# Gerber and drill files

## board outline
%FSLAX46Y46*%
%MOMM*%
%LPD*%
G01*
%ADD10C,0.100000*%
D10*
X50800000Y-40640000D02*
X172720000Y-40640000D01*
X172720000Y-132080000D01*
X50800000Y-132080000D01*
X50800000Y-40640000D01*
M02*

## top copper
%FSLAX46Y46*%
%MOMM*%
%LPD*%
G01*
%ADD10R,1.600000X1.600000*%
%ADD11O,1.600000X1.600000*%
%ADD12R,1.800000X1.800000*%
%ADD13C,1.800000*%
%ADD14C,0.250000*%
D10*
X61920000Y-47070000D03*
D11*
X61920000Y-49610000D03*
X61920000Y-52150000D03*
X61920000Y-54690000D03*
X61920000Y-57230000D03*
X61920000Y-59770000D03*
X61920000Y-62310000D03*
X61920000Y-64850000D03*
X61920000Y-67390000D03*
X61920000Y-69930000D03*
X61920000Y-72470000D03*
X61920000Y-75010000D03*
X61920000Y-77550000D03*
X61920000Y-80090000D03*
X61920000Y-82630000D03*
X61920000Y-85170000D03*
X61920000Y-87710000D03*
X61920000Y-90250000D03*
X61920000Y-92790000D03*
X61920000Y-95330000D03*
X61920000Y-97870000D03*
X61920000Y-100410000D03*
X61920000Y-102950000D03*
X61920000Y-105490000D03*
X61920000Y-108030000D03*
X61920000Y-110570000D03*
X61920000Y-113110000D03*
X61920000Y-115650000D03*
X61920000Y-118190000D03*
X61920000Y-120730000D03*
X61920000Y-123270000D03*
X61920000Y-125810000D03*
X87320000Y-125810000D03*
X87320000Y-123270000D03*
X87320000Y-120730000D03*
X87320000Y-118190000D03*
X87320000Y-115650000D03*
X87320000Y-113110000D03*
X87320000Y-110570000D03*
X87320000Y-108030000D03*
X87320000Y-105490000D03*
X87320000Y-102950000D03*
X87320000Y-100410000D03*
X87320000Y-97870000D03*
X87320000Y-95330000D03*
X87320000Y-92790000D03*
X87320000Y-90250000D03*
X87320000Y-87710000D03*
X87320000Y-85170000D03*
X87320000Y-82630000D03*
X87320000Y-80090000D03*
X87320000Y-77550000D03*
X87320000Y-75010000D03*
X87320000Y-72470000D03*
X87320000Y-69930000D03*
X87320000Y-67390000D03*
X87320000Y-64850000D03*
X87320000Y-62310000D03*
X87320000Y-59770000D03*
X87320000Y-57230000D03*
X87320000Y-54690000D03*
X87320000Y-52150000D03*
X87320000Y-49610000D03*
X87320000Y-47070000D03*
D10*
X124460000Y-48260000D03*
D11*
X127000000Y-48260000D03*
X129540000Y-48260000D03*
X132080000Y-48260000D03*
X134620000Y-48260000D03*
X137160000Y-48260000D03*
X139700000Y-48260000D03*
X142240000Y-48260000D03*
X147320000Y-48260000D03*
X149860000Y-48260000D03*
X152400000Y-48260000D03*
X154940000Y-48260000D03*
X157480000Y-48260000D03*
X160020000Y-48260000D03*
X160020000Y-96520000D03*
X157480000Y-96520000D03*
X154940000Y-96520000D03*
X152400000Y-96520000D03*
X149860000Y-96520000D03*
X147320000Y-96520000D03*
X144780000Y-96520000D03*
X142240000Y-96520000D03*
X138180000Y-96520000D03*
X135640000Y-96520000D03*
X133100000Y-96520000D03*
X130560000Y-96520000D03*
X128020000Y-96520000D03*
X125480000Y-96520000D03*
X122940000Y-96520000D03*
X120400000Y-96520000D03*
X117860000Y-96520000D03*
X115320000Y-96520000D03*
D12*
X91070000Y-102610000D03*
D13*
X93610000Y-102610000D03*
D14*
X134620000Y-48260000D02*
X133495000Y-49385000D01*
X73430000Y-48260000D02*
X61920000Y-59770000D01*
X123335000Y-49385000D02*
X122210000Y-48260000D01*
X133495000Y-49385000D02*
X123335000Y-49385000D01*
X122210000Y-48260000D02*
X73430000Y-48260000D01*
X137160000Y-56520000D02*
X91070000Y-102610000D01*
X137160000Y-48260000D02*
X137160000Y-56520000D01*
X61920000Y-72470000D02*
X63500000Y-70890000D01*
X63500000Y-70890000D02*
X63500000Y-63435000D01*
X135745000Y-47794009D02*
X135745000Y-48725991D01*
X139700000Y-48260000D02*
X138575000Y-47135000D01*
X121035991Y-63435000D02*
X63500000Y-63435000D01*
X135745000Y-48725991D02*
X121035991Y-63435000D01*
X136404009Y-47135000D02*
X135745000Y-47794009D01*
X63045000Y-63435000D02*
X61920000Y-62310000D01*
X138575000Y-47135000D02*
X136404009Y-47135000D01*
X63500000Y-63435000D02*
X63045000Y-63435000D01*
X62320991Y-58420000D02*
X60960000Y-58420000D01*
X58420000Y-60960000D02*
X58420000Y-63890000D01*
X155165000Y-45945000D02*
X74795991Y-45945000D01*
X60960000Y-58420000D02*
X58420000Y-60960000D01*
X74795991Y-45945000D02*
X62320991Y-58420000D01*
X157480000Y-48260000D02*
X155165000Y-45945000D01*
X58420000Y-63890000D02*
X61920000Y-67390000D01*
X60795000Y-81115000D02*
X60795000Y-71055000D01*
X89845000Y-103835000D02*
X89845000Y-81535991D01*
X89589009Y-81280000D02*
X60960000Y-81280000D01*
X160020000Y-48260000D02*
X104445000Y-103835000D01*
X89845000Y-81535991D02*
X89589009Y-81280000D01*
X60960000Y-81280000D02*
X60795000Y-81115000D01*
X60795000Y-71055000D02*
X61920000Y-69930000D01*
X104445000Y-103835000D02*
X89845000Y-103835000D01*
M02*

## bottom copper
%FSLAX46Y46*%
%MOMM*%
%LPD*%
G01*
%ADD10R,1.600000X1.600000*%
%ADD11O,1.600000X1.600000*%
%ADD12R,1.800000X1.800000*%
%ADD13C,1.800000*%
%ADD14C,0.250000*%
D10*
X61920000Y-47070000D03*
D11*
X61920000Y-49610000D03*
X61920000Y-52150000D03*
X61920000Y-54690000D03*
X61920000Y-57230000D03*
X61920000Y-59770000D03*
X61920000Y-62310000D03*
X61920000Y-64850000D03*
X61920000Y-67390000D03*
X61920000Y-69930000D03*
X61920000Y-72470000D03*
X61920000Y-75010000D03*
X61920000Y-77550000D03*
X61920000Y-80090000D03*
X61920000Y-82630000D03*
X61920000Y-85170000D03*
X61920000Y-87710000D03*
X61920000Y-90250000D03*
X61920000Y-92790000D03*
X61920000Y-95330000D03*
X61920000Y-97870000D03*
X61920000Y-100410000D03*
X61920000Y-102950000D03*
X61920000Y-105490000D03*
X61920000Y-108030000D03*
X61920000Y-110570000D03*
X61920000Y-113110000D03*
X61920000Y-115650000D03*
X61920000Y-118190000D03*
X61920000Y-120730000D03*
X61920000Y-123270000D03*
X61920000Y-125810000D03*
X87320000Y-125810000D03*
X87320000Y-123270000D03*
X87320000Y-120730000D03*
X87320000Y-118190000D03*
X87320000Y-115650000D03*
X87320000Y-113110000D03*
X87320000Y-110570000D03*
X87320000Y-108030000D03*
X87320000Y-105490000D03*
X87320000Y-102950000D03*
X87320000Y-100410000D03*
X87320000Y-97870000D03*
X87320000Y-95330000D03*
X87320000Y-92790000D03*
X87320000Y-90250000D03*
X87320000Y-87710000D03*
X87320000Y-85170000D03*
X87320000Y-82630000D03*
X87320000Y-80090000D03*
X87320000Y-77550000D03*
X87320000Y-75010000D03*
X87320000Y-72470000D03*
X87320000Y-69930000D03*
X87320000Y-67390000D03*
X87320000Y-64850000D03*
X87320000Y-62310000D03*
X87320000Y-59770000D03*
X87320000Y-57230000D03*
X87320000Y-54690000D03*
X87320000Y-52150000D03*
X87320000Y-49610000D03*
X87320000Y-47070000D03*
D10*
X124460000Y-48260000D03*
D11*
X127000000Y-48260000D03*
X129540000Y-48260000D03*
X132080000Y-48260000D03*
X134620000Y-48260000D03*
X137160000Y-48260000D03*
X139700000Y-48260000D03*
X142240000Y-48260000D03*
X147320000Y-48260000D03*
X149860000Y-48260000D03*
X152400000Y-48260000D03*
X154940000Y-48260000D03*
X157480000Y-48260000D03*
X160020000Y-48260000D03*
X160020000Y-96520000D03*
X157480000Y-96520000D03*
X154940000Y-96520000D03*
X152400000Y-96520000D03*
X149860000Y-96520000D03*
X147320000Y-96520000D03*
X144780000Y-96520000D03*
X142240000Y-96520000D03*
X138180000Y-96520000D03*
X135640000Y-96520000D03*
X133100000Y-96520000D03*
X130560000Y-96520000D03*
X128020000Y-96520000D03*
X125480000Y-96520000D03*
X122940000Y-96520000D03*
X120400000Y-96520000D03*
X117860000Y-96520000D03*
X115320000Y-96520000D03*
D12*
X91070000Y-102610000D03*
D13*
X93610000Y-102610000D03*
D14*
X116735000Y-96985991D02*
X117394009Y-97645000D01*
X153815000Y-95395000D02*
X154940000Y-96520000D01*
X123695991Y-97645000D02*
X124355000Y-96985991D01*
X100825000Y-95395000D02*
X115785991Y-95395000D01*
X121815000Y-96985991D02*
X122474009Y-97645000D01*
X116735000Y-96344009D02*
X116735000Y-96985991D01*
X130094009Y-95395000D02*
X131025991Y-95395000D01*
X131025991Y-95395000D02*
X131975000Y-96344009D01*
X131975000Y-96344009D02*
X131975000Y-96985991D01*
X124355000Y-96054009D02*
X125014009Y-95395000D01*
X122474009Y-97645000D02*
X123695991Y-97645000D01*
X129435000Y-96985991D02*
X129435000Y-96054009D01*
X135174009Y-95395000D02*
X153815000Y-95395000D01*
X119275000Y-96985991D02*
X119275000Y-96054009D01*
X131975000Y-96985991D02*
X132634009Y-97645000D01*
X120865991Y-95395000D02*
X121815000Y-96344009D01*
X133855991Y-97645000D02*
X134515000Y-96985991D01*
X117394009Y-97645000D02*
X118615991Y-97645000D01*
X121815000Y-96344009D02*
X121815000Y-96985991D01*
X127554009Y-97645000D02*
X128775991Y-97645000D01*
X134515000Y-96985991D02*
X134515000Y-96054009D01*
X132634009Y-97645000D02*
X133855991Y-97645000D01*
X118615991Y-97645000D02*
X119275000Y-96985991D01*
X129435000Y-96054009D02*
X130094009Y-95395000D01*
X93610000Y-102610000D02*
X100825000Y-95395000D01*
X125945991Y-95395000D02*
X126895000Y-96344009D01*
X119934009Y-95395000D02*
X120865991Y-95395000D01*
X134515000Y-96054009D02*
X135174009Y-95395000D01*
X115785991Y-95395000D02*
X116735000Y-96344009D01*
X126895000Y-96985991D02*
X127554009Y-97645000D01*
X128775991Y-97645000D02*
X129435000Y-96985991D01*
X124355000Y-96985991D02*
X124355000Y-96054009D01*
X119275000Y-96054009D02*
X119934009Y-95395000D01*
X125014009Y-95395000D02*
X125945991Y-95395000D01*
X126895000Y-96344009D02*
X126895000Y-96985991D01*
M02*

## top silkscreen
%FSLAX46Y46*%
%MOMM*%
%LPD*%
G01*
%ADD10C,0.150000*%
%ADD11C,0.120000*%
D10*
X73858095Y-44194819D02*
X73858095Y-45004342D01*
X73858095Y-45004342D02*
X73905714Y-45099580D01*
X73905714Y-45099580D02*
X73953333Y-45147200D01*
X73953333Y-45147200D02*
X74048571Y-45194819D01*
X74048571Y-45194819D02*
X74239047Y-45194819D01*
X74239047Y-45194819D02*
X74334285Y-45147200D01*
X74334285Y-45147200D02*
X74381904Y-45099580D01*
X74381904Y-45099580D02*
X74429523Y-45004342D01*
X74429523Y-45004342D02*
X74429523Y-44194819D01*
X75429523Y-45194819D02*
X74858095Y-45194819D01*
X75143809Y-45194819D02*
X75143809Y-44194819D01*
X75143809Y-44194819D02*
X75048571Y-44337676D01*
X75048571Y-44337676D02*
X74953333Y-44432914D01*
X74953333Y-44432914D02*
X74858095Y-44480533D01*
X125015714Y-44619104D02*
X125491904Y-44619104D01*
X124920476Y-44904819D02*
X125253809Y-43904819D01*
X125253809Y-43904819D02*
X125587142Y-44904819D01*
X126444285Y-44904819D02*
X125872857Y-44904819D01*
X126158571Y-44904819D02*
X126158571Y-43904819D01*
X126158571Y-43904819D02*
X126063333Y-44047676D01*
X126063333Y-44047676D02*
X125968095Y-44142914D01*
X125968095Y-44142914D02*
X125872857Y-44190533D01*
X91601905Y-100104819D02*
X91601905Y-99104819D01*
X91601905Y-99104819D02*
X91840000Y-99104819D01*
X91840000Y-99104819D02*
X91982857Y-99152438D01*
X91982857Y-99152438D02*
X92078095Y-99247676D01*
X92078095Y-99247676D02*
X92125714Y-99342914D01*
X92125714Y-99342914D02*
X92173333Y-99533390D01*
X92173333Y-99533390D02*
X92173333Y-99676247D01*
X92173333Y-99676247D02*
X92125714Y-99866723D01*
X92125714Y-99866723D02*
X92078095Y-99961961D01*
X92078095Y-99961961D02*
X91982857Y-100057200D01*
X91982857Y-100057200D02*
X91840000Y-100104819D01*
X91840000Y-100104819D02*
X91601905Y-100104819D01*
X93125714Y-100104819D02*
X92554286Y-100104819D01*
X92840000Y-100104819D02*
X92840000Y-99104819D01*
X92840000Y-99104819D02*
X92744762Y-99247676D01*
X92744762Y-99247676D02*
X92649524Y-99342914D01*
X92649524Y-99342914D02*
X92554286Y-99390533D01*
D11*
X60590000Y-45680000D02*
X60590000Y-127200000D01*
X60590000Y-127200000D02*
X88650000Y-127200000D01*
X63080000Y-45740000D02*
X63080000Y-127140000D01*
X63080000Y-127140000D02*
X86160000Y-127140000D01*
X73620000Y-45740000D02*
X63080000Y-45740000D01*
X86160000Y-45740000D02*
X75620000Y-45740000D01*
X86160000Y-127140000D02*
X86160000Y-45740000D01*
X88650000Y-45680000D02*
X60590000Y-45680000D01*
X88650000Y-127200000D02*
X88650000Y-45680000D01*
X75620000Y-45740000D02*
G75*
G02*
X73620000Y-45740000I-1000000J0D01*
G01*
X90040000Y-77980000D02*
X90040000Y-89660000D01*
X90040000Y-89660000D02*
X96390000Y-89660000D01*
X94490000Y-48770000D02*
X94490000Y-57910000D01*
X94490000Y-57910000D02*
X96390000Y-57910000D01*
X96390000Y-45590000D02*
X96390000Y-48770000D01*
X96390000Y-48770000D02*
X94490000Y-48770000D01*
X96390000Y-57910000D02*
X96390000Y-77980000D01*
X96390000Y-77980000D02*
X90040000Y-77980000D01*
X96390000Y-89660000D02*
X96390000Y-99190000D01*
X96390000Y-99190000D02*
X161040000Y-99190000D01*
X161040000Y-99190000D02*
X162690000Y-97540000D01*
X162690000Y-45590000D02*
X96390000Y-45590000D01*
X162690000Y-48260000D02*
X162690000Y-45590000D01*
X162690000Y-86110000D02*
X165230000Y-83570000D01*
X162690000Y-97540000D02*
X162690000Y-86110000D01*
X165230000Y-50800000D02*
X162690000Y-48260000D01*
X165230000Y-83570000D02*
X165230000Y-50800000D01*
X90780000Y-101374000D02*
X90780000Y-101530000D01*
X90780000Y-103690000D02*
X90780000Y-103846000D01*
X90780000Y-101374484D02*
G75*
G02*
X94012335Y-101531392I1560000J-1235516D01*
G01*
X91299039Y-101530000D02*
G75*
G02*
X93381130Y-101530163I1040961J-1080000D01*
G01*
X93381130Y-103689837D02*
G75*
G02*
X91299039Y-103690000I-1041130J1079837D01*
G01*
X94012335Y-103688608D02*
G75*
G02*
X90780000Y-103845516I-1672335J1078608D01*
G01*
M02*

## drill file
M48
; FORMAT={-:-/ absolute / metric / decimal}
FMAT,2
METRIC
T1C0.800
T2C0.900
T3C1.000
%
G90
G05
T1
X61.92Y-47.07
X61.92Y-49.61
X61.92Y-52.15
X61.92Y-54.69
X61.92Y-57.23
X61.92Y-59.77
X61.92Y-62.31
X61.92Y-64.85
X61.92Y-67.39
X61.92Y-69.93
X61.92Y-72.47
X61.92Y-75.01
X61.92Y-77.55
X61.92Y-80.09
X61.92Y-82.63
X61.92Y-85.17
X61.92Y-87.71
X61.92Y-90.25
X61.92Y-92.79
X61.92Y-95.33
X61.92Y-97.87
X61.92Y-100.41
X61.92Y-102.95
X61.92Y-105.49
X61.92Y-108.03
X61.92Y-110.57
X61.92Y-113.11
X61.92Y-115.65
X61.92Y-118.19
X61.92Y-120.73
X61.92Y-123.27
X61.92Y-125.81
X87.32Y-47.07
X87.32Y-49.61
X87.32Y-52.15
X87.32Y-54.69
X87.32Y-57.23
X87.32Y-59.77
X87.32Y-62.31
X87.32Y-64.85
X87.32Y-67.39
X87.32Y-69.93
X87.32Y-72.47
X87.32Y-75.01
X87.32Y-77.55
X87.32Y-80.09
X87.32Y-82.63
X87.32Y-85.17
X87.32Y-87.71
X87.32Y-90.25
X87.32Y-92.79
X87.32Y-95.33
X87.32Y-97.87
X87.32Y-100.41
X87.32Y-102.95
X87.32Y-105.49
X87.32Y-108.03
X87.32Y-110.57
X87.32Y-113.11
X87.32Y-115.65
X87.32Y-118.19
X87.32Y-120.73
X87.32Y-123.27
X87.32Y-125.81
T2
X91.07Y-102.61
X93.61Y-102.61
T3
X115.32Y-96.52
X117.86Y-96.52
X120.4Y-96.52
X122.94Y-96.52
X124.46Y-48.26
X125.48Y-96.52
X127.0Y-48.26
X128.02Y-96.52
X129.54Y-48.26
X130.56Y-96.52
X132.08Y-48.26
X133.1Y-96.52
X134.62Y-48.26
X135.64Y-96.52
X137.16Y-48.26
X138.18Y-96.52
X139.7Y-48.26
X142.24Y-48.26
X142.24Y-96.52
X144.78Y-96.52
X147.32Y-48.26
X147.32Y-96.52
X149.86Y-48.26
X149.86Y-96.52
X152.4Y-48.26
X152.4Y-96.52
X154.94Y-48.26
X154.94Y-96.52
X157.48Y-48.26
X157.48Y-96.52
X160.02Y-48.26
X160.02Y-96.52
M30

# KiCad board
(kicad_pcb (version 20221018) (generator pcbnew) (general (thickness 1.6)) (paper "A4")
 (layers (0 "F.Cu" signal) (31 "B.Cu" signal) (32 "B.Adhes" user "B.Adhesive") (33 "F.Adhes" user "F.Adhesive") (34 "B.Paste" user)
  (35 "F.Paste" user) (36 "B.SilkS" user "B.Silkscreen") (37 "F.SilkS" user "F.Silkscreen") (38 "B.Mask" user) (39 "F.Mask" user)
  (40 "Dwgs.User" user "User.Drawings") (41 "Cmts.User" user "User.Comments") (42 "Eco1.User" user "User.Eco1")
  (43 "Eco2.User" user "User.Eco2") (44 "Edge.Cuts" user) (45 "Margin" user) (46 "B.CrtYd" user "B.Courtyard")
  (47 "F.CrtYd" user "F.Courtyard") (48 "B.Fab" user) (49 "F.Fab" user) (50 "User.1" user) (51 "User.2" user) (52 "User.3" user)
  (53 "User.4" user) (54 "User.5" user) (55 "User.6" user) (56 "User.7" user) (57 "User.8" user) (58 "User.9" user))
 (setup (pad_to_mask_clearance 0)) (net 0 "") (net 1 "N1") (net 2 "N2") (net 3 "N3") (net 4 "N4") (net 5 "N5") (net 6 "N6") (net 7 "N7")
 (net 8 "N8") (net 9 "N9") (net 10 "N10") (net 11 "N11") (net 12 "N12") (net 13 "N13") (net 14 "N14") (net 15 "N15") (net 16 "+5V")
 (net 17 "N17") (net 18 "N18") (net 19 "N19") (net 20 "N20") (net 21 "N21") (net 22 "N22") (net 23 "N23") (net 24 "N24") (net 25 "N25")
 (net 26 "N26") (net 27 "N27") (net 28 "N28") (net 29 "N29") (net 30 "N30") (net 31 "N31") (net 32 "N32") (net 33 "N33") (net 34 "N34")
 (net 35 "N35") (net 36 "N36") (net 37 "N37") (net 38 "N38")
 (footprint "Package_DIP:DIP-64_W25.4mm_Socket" (layer "F.Cu") (at 61.92 47.07)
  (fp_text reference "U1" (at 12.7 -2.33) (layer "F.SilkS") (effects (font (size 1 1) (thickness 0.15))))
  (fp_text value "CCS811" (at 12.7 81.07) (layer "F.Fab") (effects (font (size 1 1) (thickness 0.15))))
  (fp_line (start -1.33 -1.39) (end -1.33 80.13) (stroke (width 0.12) (type solid)) (layer "F.SilkS"))
  (fp_line (start -1.33 80.13) (end 26.73 80.13) (stroke (width 0.12) (type solid)) (layer "F.SilkS"))
  (fp_line (start 1.16 -1.33) (end 1.16 80.07) (stroke (width 0.12) (type solid)) (layer "F.SilkS"))
  (fp_line (start 1.16 80.07) (end 24.24 80.07) (stroke (width 0.12) (type solid)) (layer "F.SilkS"))
  (fp_line (start 11.7 -1.33) (end 1.16 -1.33) (stroke (width 0.12) (type solid)) (layer "F.SilkS"))
  (fp_line (start 24.24 -1.33) (end 13.7 -1.33) (stroke (width 0.12) (type solid)) (layer "F.SilkS"))
  (fp_line (start 24.24 80.07) (end 24.24 -1.33) (stroke (width 0.12) (type solid)) (layer "F.SilkS"))
  (fp_line (start 26.73 -1.39) (end -1.33 -1.39) (stroke (width 0.12) (type solid)) (layer "F.SilkS"))
  (fp_line (start 26.73 80.13) (end 26.73 -1.39) (stroke (width 0.12) (type solid)) (layer "F.SilkS"))
  (fp_arc (start 13.7 -1.33) (mid 12.7 -0.33) (end 11.7 -1.33) (stroke (width 0.12) (type solid)) (layer "F.SilkS"))
  (pad "1" thru_hole rect (at 0 0) (size 1.6 1.6) (drill 0.8) (layers "*.Cu" "*.Mask") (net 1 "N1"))
  (pad "2" thru_hole oval (at 0 2.54) (size 1.6 1.6) (drill 0.8) (layers "*.Cu" "*.Mask") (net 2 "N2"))
  (pad "3" thru_hole oval (at 0 5.08) (size 1.6 1.6) (drill 0.8) (layers "*.Cu" "*.Mask") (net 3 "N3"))
  (pad "4" thru_hole oval (at 0 7.62) (size 1.6 1.6) (drill 0.8) (layers "*.Cu" "*.Mask") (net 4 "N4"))
  (pad "5" thru_hole oval (at 0 10.16) (size 1.6 1.6) (drill 0.8) (layers "*.Cu" "*.Mask") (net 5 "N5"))
  (pad "6" thru_hole oval (at 0 12.7) (size 1.6 1.6) (drill 0.8) (layers "*.Cu" "*.Mask") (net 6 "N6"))
  (pad "7" thru_hole oval (at 0 15.24) (size 1.6 1.6) (drill 0.8) (layers "*.Cu" "*.Mask") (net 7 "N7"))
  (pad "8" thru_hole oval (at 0 17.78) (size 1.6 1.6) (drill 0.8) (layers "*.Cu" "*.Mask") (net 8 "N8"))
  (pad "9" thru_hole oval (at 0 20.32) (size 1.6 1.6) (drill 0.8) (layers "*.Cu" "*.Mask") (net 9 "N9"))
  (pad "10" thru_hole oval (at 0 22.86) (size 1.6 1.6) (drill 0.8) (layers "*.Cu" "*.Mask") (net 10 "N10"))
  (pad "11" thru_hole oval (at 0 25.4) (size 1.6 1.6) (drill 0.8) (layers "*.Cu" "*.Mask") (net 7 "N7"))
  (pad "12" thru_hole oval (at 0 27.94) (size 1.6 1.6) (drill 0.8) (layers "*.Cu" "*.Mask"))
  (pad "13" thru_hole oval (at 0 30.48) (size 1.6 1.6) (drill 0.8) (layers "*.Cu" "*.Mask"))
  (pad "14" thru_hole oval (at 0 33.02) (size 1.6 1.6) (drill 0.8) (layers "*.Cu" "*.Mask"))
  (pad "15" thru_hole oval (at 0 35.56) (size 1.6 1.6) (drill 0.8) (layers "*.Cu" "*.Mask"))
  (pad "16" thru_hole oval (at 0 38.1) (size 1.6 1.6) (drill 0.8) (layers "*.Cu" "*.Mask"))
  (pad "17" thru_hole oval (at 0 40.64) (size 1.6 1.6) (drill 0.8) (layers "*.Cu" "*.Mask"))
  (pad "18" thru_hole oval (at 0 43.18) (size 1.6 1.6) (drill 0.8) (layers "*.Cu" "*.Mask"))
  (pad "19" thru_hole oval (at 0 45.72) (size 1.6 1.6) (drill 0.8) (layers "*.Cu" "*.Mask"))
  (pad "20" thru_hole oval (at 0 48.26) (size 1.6 1.6) (drill 0.8) (layers "*.Cu" "*.Mask"))
  (pad "21" thru_hole oval (at 0 50.8) (size 1.6 1.6) (drill 0.8) (layers "*.Cu" "*.Mask"))
  (pad "22" thru_hole oval (at 0 53.34) (size 1.6 1.6) (drill 0.8) (layers "*.Cu" "*.Mask"))
  (pad "23" thru_hole oval (at 0 55.88) (size 1.6 1.6) (drill 0.8) (layers "*.Cu" "*.Mask"))
  (pad "24" thru_hole oval (at 0 58.42) (size 1.6 1.6) (drill 0.8) (layers "*.Cu" "*.Mask"))
  (pad "25" thru_hole oval (at 0 60.96) (size 1.6 1.6) (drill 0.8) (layers "*.Cu" "*.Mask"))
  (pad "26" thru_hole oval (at 0 63.5) (size 1.6 1.6) (drill 0.8) (layers "*.Cu" "*.Mask"))
  (pad "27" thru_hole oval (at 0 66.04) (size 1.6 1.6) (drill 0.8) (layers "*.Cu" "*.Mask"))
  (pad "28" thru_hole oval (at 0 68.58) (size 1.6 1.6) (drill 0.8) (layers "*.Cu" "*.Mask"))
  (pad "29" thru_hole oval (at 0 71.12) (size 1.6 1.6) (drill 0.8) (layers "*.Cu" "*.Mask"))
  (pad "30" thru_hole oval (at 0 73.66) (size 1.6 1.6) (drill 0.8) (layers "*.Cu" "*.Mask"))
  (pad "31" thru_hole oval (at 0 76.2) (size 1.6 1.6) (drill 0.8) (layers "*.Cu" "*.Mask"))
  (pad "32" thru_hole oval (at 0 78.74) (size 1.6 1.6) (drill 0.8) (layers "*.Cu" "*.Mask"))
  (pad "33" thru_hole oval (at 25.4 78.74) (size 1.6 1.6) (drill 0.8) (layers "*.Cu" "*.Mask"))
  (pad "34" thru_hole oval (at 25.4 76.2) (size 1.6 1.6) (drill 0.8) (layers "*.Cu" "*.Mask"))
  (pad "35" thru_hole oval (at 25.4 73.66) (size 1.6 1.6) (drill 0.8) (layers "*.Cu" "*.Mask"))
  (pad "36" thru_hole oval (at 25.4 71.12) (size 1.6 1.6) (drill 0.8) (layers "*.Cu" "*.Mask"))
  (pad "37" thru_hole oval (at 25.4 68.58) (size 1.6 1.6) (drill 0.8) (layers "*.Cu" "*.Mask"))
  (pad "38" thru_hole oval (at 25.4 66.04) (size 1.6 1.6) (drill 0.8) (layers "*.Cu" "*.Mask"))
  (pad "39" thru_hole oval (at 25.4 63.5) (size 1.6 1.6) (drill 0.8) (layers "*.Cu" "*.Mask"))
  (pad "40" thru_hole oval (at 25.4 60.96) (size 1.6 1.6) (drill 0.8) (layers "*.Cu" "*.Mask"))
  (pad "41" thru_hole oval (at 25.4 58.42) (size 1.6 1.6) (drill 0.8) (layers "*.Cu" "*.Mask"))
  (pad "42" thru_hole oval (at 25.4 55.88) (size 1.6 1.6) (drill 0.8) (layers "*.Cu" "*.Mask"))
  (pad "43" thru_hole oval (at 25.4 53.34) (size 1.6 1.6) (drill 0.8) (layers "*.Cu" "*.Mask"))
  (pad "44" thru_hole oval (at 25.4 50.8) (size 1.6 1.6) (drill 0.8) (layers "*.Cu" "*.Mask"))
  (pad "45" thru_hole oval (at 25.4 48.26) (size 1.6 1.6) (drill 0.8) (layers "*.Cu" "*.Mask"))
  (pad "46" thru_hole oval (at 25.4 45.72) (size 1.6 1.6) (drill 0.8) (layers "*.Cu" "*.Mask"))
  (pad "47" thru_hole oval (at 25.4 43.18) (size 1.6 1.6) (drill 0.8) (layers "*.Cu" "*.Mask"))
  (pad "48" thru_hole oval (at 25.4 40.64) (size 1.6 1.6) (drill 0.8) (layers "*.Cu" "*.Mask"))
  (pad "49" thru_hole oval (at 25.4 38.1) (size 1.6 1.6) (drill 0.8) (layers "*.Cu" "*.Mask"))
  (pad "50" thru_hole oval (at 25.4 35.56) (size 1.6 1.6) (drill 0.8) (layers "*.Cu" "*.Mask"))
  (pad "51" thru_hole oval (at 25.4 33.02) (size 1.6 1.6) (drill 0.8) (layers "*.Cu" "*.Mask"))
  (pad "52" thru_hole oval (at 25.4 30.48) (size 1.6 1.6) (drill 0.8) (layers "*.Cu" "*.Mask"))
  (pad "53" thru_hole oval (at 25.4 27.94) (size 1.6 1.6) (drill 0.8) (layers "*.Cu" "*.Mask"))
  (pad "54" thru_hole oval (at 25.4 25.4) (size 1.6 1.6) (drill 0.8) (layers "*.Cu" "*.Mask"))
  (pad "55" thru_hole oval (at 25.4 22.86) (size 1.6 1.6) (drill 0.8) (layers "*.Cu" "*.Mask"))
  (pad "56" thru_hole oval (at 25.4 20.32) (size 1.6 1.6) (drill 0.8) (layers "*.Cu" "*.Mask"))
  (pad "57" thru_hole oval (at 25.4 17.78) (size 1.6 1.6) (drill 0.8) (layers "*.Cu" "*.Mask"))
  (pad "58" thru_hole oval (at 25.4 15.24) (size 1.6 1.6) (drill 0.8) (layers "*.Cu" "*.Mask"))
  (pad "59" thru_hole oval (at 25.4 12.7) (size 1.6 1.6) (drill 0.8) (layers "*.Cu" "*.Mask"))
  (pad "60" thru_hole oval (at 25.4 10.16) (size 1.6 1.6) (drill 0.8) (layers "*.Cu" "*.Mask"))
  (pad "61" thru_hole oval (at 25.4 7.62) (size 1.6 1.6) (drill 0.8) (layers "*.Cu" "*.Mask"))
  (pad "62" thru_hole oval (at 25.4 5.08) (size 1.6 1.6) (drill 0.8) (layers "*.Cu" "*.Mask"))
  (pad "63" thru_hole oval (at 25.4 2.54) (size 1.6 1.6) (drill 0.8) (layers "*.Cu" "*.Mask"))
  (pad "64" thru_hole oval (at 25.4 0) (size 1.6 1.6) (drill 0.8) (layers "*.Cu" "*.Mask")))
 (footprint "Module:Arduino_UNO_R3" (layer "F.Cu") (at 124.46 48.26)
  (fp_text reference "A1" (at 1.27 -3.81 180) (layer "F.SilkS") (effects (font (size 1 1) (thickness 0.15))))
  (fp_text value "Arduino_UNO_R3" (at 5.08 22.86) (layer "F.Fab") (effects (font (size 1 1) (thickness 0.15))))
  (fp_line (start -34.42 29.72) (end -34.42 41.4) (stroke (width 0.12) (type solid)) (layer "F.SilkS"))
  (fp_line (start -34.42 41.4) (end -28.07 41.4) (stroke (width 0.12) (type solid)) (layer "F.SilkS"))
  (fp_line (start -29.97 0.51) (end -29.97 9.65) (stroke (width 0.12) (type solid)) (layer "F.SilkS"))
  (fp_line (start -29.97 9.65) (end -28.07 9.65) (stroke (width 0.12) (type solid)) (layer "F.SilkS"))
  (fp_line (start -28.07 -2.67) (end -28.07 0.51) (stroke (width 0.12) (type solid)) (layer "F.SilkS"))
  (fp_line (start -28.07 0.51) (end -29.97 0.51) (stroke (width 0.12) (type solid)) (layer "F.SilkS"))
  (fp_line (start -28.07 9.65) (end -28.07 29.72) (stroke (width 0.12) (type solid)) (layer "F.SilkS"))
  (fp_line (start -28.07 29.72) (end -34.42 29.72) (stroke (width 0.12) (type solid)) (layer "F.SilkS"))
  (fp_line (start -28.07 41.4) (end -28.07 50.93) (stroke (width 0.12) (type solid)) (layer "F.SilkS"))
  (fp_line (start -28.07 50.93) (end 36.58 50.93) (stroke (width 0.12) (type solid)) (layer "F.SilkS"))
  (fp_line (start 36.58 50.93) (end 38.23 49.28) (stroke (width 0.12) (type solid)) (layer "F.SilkS"))
  (fp_line (start 38.23 -2.67) (end -28.07 -2.67) (stroke (width 0.12) (type solid)) (layer "F.SilkS"))
  (fp_line (start 38.23 0) (end 38.23 -2.67) (stroke (width 0.12) (type solid)) (layer "F.SilkS"))
  (fp_line (start 38.23 37.85) (end 40.77 35.31) (stroke (width 0.12) (type solid)) (layer "F.SilkS"))
  (fp_line (start 38.23 49.28) (end 38.23 37.85) (stroke (width 0.12) (type solid)) (layer "F.SilkS"))
  (fp_line (start 40.77 2.54) (end 38.23 0) (stroke (width 0.12) (type solid)) (layer "F.SilkS"))
  (fp_line (start 40.77 35.31) (end 40.77 2.54) (stroke (width 0.12) (type solid)) (layer "F.SilkS"))
  (pad "1" thru_hole rect (at 0 0 90) (size 1.6 1.6) (drill 1) (layers "*.Cu" "*.Mask") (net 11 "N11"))
  (pad "2" thru_hole oval (at 2.54 0 90) (size 1.6 1.6) (drill 1) (layers "*.Cu" "*.Mask") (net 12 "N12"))
  (pad "3" thru_hole oval (at 5.08 0 90) (size 1.6 1.6) (drill 1) (layers "*.Cu" "*.Mask") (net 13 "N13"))
  (pad "4" thru_hole oval (at 7.62 0 90) (size 1.6 1.6) (drill 1) (layers "*.Cu" "*.Mask") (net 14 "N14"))
  (pad "5" thru_hole oval (at 10.16 0 90) (size 1.6 1.6) (drill 1) (layers "*.Cu" "*.Mask") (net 6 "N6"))
  (pad "6" thru_hole oval (at 12.7 0 90) (size 1.6 1.6) (drill 1) (layers "*.Cu" "*.Mask") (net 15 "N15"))
  (pad "7" thru_hole oval (at 15.24 0 90) (size 1.6 1.6) (drill 1) (layers "*.Cu" "*.Mask") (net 7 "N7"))
  (pad "8" thru_hole oval (at 17.78 0 90) (size 1.6 1.6) (drill 1) (layers "*.Cu" "*.Mask") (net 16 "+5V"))
  (pad "9" thru_hole oval (at 22.86 0 90) (size 1.6 1.6) (drill 1) (layers "*.Cu" "*.Mask") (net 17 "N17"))
  (pad "10" thru_hole oval (at 25.4 0 90) (size 1.6 1.6) (drill 1) (layers "*.Cu" "*.Mask") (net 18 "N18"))
  (pad "11" thru_hole oval (at 27.94 0 90) (size 1.6 1.6) (drill 1) (layers "*.Cu" "*.Mask") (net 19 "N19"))
  (pad "12" thru_hole oval (at 30.48 0 90) (size 1.6 1.6) (drill 1) (layers "*.Cu" "*.Mask") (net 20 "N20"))
  (pad "13" thru_hole oval (at 33.02 0 90) (size 1.6 1.6) (drill 1) (layers "*.Cu" "*.Mask") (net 9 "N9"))
  (pad "14" thru_hole oval (at 35.56 0 90) (size 1.6 1.6) (drill 1) (layers "*.Cu" "*.Mask") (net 10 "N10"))
  (pad "15" thru_hole oval (at 35.56 48.26 90) (size 1.6 1.6) (drill 1) (layers "*.Cu" "*.Mask") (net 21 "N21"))
  (pad "16" thru_hole oval (at 33.02 48.26 90) (size 1.6 1.6) (drill 1) (layers "*.Cu" "*.Mask") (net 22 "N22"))
  (pad "17" thru_hole oval (at 30.48 48.26 90) (size 1.6 1.6) (drill 1) (layers "*.Cu" "*.Mask") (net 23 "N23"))
  (pad "18" thru_hole oval (at 27.94 48.26 90) (size 1.6 1.6) (drill 1) (layers "*.Cu" "*.Mask") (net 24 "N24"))
  (pad "19" thru_hole oval (at 25.4 48.26 90) (size 1.6 1.6) (drill 1) (layers "*.Cu" "*.Mask") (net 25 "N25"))
  (pad "20" thru_hole oval (at 22.86 48.26 90) (size 1.6 1.6) (drill 1) (layers "*.Cu" "*.Mask") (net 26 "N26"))
  (pad "21" thru_hole oval (at 20.32 48.26 90) (size 1.6 1.6) (drill 1) (layers "*.Cu" "*.Mask") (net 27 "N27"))
  (pad "22" thru_hole oval (at 17.78 48.26 90) (size 1.6 1.6) (drill 1) (layers "*.Cu" "*.Mask") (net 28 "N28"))
  (pad "23" thru_hole oval (at 13.72 48.26 90) (size 1.6 1.6) (drill 1) (layers "*.Cu" "*.Mask") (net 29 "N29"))
  (pad "24" thru_hole oval (at 11.18 48.26 90) (size 1.6 1.6) (drill 1) (layers "*.Cu" "*.Mask") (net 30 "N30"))
  (pad "25" thru_hole oval (at 8.64 48.26 90) (size 1.6 1.6) (drill 1) (layers "*.Cu" "*.Mask") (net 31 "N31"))
  (pad "26" thru_hole oval (at 6.1 48.26 90) (size 1.6 1.6) (drill 1) (layers "*.Cu" "*.Mask") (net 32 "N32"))
  (pad "27" thru_hole oval (at 3.56 48.26 90) (size 1.6 1.6) (drill 1) (layers "*.Cu" "*.Mask") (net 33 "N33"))
  (pad "28" thru_hole oval (at 1.02 48.26 90) (size 1.6 1.6) (drill 1) (layers "*.Cu" "*.Mask") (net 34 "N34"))
  (pad "29" thru_hole oval (at -1.52 48.26 90) (size 1.6 1.6) (drill 1) (layers "*.Cu" "*.Mask") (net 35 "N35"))
  (pad "30" thru_hole oval (at -4.06 48.26 90) (size 1.6 1.6) (drill 1) (layers "*.Cu" "*.Mask") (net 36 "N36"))
  (pad "31" thru_hole oval (at -6.6 48.26 90) (size 1.6 1.6) (drill 1) (layers "*.Cu" "*.Mask") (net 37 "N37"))
  (pad "32" thru_hole oval (at -9.14 48.26 90) (size 1.6 1.6) (drill 1) (layers "*.Cu" "*.Mask") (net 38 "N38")))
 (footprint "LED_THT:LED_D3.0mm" (layer "F.Cu") (at 91.07 102.61)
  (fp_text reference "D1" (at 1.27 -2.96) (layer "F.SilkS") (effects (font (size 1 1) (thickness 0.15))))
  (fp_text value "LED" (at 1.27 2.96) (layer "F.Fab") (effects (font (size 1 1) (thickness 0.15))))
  (fp_line (start -0.29 -1.236) (end -0.29 -1.08) (stroke (width 0.12) (type solid)) (layer "F.SilkS"))
  (fp_line (start -0.29 1.08) (end -0.29 1.236) (stroke (width 0.12) (type solid)) (layer "F.SilkS"))
  (fp_arc (start -0.29 -1.235516) (mid 1.366487 -1.987659) (end 2.942335 -1.078608) (stroke (width 0.12) (type solid)) (layer "F.SilkS"))
  (fp_arc (start 0.229039 -1.08) (mid 1.270117 -1.5) (end 2.31113 -1.079837) (stroke (width 0.12) (type solid)) (layer "F.SilkS"))
  (fp_arc (start 2.31113 1.079837) (mid 1.270117 1.5) (end 0.229039 1.08) (stroke (width 0.12) (type solid)) (layer "F.SilkS"))
  (fp_arc (start 2.942335 1.078608) (mid 1.366487 1.987659) (end -0.29 1.235516) (stroke (width 0.12) (type solid)) (layer "F.SilkS"))
  (pad "1" thru_hole rect (at 0 0) (size 1.8 1.8) (drill 0.9) (layers "*.Cu" "*.Mask") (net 15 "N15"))
  (pad "2" thru_hole circle (at 2.54 0) (size 1.8 1.8) (drill 0.9) (layers "*.Cu" "*.Mask") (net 23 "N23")))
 (gr_rect (start 50.8 40.64) (end 172.72 132.08) (stroke (width 0.1) (type default)) (fill none) (layer "Edge.Cuts"))
 (segment (start 134.62 48.26) (end 133.495 49.385) (width 0.25) (layer "F.Cu") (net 6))
 (segment (start 73.43 48.26) (end 61.92 59.77) (width 0.25) (layer "F.Cu") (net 6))
 (segment (start 123.335 49.385) (end 122.21 48.26) (width 0.25) (layer "F.Cu") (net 6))
 (segment (start 133.495 49.385) (end 123.335 49.385) (width 0.25) (layer "F.Cu") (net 6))
 (segment (start 122.21 48.26) (end 73.43 48.26) (width 0.25) (layer "F.Cu") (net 6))
 (segment (start 137.16 56.52) (end 91.07 102.61) (width 0.25) (layer "F.Cu") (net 15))
 (segment (start 137.16 48.26) (end 137.16 56.52) (width 0.25) (layer "F.Cu") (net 15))
 (segment (start 61.92 72.47) (end 63.5 70.89) (width 0.25) (layer "F.Cu") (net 7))
 (segment (start 63.5 70.89) (end 63.5 63.435) (width 0.25) (layer "F.Cu") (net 7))
 (segment (start 135.745 47.794009) (end 135.745 48.725991) (width 0.25) (layer "F.Cu") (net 7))
 (segment (start 139.7 48.26) (end 138.575 47.135) (width 0.25) (layer "F.Cu") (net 7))
 (segment (start 121.035991 63.435) (end 63.5 63.435) (width 0.25) (layer "F.Cu") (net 7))
 (segment (start 135.745 48.725991) (end 121.035991 63.435) (width 0.25) (layer "F.Cu") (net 7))
 (segment (start 136.404009 47.135) (end 135.745 47.794009) (width 0.25) (layer "F.Cu") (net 7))
 (segment (start 63.045 63.435) (end 61.92 62.31) (width 0.25) (layer "F.Cu") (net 7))
 (segment (start 138.575 47.135) (end 136.404009 47.135) (width 0.25) (layer "F.Cu") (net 7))
 (segment (start 63.5 63.435) (end 63.045 63.435) (width 0.25) (layer "F.Cu") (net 7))
 (segment (start 62.320991 58.42) (end 60.96 58.42) (width 0.25) (layer "F.Cu") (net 9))
 (segment (start 58.42 60.96) (end 58.42 63.89) (width 0.25) (layer "F.Cu") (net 9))
 (segment (start 155.165 45.945) (end 74.795991 45.945) (width 0.25) (layer "F.Cu") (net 9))
 (segment (start 60.96 58.42) (end 58.42 60.96) (width 0.25) (layer "F.Cu") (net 9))
 (segment (start 74.795991 45.945) (end 62.320991 58.42) (width 0.25) (layer "F.Cu") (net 9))
 (segment (start 157.48 48.26) (end 155.165 45.945) (width 0.25) (layer "F.Cu") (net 9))
 (segment (start 58.42 63.89) (end 61.92 67.39) (width 0.25) (layer "F.Cu") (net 9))
 (segment (start 60.795 81.115) (end 60.795 71.055) (width 0.25) (layer "F.Cu") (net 10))
 (segment (start 89.845 103.835) (end 89.845 81.535991) (width 0.25) (layer "F.Cu") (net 10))
 (segment (start 89.589009 81.28) (end 60.96 81.28) (width 0.25) (layer "F.Cu") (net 10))
 (segment (start 160.02 48.26) (end 104.445 103.835) (width 0.25) (layer "F.Cu") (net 10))
 (segment (start 89.845 81.535991) (end 89.589009 81.28) (width 0.25) (layer "F.Cu") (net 10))
 (segment (start 60.96 81.28) (end 60.795 81.115) (width 0.25) (layer "F.Cu") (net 10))
 (segment (start 60.795 71.055) (end 61.92 69.93) (width 0.25) (layer "F.Cu") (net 10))
 (segment (start 104.445 103.835) (end 89.845 103.835) (width 0.25) (layer "F.Cu") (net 10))
 (segment (start 116.735 96.985991) (end 117.394009 97.645) (width 0.25) (layer "B.Cu") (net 23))
 (segment (start 153.815 95.395) (end 154.94 96.52) (width 0.25) (layer "B.Cu") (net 23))
 (segment (start 123.695991 97.645) (end 124.355 96.985991) (width 0.25) (layer "B.Cu") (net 23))
 (segment (start 100.825 95.395) (end 115.785991 95.395) (width 0.25) (layer "B.Cu") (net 23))
 (segment (start 121.815 96.985991) (end 122.474009 97.645) (width 0.25) (layer "B.Cu") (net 23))
 (segment (start 116.735 96.344009) (end 116.735 96.985991) (width 0.25) (layer "B.Cu") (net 23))
 (segment (start 130.094009 95.395) (end 131.025991 95.395) (width 0.25) (layer "B.Cu") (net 23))
 (segment (start 131.025991 95.395) (end 131.975 96.344009) (width 0.25) (layer "B.Cu") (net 23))
 (segment (start 131.975 96.344009) (end 131.975 96.985991) (width 0.25) (layer "B.Cu") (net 23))
 (segment (start 124.355 96.054009) (end 125.014009 95.395) (width 0.25) (layer "B.Cu") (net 23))
 (segment (start 122.474009 97.645) (end 123.695991 97.645) (width 0.25) (layer "B.Cu") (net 23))
 (segment (start 129.435 96.985991) (end 129.435 96.054009) (width 0.25) (layer "B.Cu") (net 23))
 (segment (start 135.174009 95.395) (end 153.815 95.395) (width 0.25) (layer "B.Cu") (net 23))
 (segment (start 119.275 96.985991) (end 119.275 96.054009) (width 0.25) (layer "B.Cu") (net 23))
 (segment (start 131.975 96.985991) (end 132.634009 97.645) (width 0.25) (layer "B.Cu") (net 23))
 (segment (start 120.865991 95.395) (end 121.815 96.344009) (width 0.25) (layer "B.Cu") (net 23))
 (segment (start 133.855991 97.645) (end 134.515 96.985991) (width 0.25) (layer "B.Cu") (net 23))
 (segment (start 117.394009 97.645) (end 118.615991 97.645) (width 0.25) (layer "B.Cu") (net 23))
 (segment (start 121.815 96.344009) (end 121.815 96.985991) (width 0.25) (layer "B.Cu") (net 23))
 (segment (start 127.554009 97.645) (end 128.775991 97.645) (width 0.25) (layer "B.Cu") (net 23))
 (segment (start 134.515 96.985991) (end 134.515 96.054009) (width 0.25) (layer "B.Cu") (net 23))
 (segment (start 132.634009 97.645) (end 133.855991 97.645) (width 0.25) (layer "B.Cu") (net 23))
 (segment (start 118.615991 97.645) (end 119.275 96.985991) (width 0.25) (layer "B.Cu") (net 23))
 (segment (start 129.435 96.054009) (end 130.094009 95.395) (width 0.25) (layer "B.Cu") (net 23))
 (segment (start 93.61 102.61) (end 100.825 95.395) (width 0.25) (layer "B.Cu") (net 23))
 (segment (start 125.945991 95.395) (end 126.895 96.344009) (width 0.25) (layer "B.Cu") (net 23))
 (segment (start 119.934009 95.395) (end 120.865991 95.395) (width 0.25) (layer "B.Cu") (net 23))
 (segment (start 134.515 96.054009) (end 135.174009 95.395) (width 0.25) (layer "B.Cu") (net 23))
 (segment (start 115.785991 95.395) (end 116.735 96.344009) (width 0.25) (layer "B.Cu") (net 23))
 (segment (start 126.895 96.985991) (end 127.554009 97.645) (width 0.25) (layer "B.Cu") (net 23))
 (segment (start 128.775991 97.645) (end 129.435 96.985991) (width 0.25) (layer "B.Cu") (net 23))
 (segment (start 124.355 96.985991) (end 124.355 96.054009) (width 0.25) (layer "B.Cu") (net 23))
 (segment (start 119.275 96.054009) (end 119.934009 95.395) (width 0.25) (layer "B.Cu") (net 23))
 (segment (start 125.014009 95.395) (end 125.945991 95.395) (width 0.25) (layer "B.Cu") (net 23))
 (segment (start 126.895 96.344009) (end 126.895 96.985991) (width 0.25) (layer "B.Cu") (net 23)))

